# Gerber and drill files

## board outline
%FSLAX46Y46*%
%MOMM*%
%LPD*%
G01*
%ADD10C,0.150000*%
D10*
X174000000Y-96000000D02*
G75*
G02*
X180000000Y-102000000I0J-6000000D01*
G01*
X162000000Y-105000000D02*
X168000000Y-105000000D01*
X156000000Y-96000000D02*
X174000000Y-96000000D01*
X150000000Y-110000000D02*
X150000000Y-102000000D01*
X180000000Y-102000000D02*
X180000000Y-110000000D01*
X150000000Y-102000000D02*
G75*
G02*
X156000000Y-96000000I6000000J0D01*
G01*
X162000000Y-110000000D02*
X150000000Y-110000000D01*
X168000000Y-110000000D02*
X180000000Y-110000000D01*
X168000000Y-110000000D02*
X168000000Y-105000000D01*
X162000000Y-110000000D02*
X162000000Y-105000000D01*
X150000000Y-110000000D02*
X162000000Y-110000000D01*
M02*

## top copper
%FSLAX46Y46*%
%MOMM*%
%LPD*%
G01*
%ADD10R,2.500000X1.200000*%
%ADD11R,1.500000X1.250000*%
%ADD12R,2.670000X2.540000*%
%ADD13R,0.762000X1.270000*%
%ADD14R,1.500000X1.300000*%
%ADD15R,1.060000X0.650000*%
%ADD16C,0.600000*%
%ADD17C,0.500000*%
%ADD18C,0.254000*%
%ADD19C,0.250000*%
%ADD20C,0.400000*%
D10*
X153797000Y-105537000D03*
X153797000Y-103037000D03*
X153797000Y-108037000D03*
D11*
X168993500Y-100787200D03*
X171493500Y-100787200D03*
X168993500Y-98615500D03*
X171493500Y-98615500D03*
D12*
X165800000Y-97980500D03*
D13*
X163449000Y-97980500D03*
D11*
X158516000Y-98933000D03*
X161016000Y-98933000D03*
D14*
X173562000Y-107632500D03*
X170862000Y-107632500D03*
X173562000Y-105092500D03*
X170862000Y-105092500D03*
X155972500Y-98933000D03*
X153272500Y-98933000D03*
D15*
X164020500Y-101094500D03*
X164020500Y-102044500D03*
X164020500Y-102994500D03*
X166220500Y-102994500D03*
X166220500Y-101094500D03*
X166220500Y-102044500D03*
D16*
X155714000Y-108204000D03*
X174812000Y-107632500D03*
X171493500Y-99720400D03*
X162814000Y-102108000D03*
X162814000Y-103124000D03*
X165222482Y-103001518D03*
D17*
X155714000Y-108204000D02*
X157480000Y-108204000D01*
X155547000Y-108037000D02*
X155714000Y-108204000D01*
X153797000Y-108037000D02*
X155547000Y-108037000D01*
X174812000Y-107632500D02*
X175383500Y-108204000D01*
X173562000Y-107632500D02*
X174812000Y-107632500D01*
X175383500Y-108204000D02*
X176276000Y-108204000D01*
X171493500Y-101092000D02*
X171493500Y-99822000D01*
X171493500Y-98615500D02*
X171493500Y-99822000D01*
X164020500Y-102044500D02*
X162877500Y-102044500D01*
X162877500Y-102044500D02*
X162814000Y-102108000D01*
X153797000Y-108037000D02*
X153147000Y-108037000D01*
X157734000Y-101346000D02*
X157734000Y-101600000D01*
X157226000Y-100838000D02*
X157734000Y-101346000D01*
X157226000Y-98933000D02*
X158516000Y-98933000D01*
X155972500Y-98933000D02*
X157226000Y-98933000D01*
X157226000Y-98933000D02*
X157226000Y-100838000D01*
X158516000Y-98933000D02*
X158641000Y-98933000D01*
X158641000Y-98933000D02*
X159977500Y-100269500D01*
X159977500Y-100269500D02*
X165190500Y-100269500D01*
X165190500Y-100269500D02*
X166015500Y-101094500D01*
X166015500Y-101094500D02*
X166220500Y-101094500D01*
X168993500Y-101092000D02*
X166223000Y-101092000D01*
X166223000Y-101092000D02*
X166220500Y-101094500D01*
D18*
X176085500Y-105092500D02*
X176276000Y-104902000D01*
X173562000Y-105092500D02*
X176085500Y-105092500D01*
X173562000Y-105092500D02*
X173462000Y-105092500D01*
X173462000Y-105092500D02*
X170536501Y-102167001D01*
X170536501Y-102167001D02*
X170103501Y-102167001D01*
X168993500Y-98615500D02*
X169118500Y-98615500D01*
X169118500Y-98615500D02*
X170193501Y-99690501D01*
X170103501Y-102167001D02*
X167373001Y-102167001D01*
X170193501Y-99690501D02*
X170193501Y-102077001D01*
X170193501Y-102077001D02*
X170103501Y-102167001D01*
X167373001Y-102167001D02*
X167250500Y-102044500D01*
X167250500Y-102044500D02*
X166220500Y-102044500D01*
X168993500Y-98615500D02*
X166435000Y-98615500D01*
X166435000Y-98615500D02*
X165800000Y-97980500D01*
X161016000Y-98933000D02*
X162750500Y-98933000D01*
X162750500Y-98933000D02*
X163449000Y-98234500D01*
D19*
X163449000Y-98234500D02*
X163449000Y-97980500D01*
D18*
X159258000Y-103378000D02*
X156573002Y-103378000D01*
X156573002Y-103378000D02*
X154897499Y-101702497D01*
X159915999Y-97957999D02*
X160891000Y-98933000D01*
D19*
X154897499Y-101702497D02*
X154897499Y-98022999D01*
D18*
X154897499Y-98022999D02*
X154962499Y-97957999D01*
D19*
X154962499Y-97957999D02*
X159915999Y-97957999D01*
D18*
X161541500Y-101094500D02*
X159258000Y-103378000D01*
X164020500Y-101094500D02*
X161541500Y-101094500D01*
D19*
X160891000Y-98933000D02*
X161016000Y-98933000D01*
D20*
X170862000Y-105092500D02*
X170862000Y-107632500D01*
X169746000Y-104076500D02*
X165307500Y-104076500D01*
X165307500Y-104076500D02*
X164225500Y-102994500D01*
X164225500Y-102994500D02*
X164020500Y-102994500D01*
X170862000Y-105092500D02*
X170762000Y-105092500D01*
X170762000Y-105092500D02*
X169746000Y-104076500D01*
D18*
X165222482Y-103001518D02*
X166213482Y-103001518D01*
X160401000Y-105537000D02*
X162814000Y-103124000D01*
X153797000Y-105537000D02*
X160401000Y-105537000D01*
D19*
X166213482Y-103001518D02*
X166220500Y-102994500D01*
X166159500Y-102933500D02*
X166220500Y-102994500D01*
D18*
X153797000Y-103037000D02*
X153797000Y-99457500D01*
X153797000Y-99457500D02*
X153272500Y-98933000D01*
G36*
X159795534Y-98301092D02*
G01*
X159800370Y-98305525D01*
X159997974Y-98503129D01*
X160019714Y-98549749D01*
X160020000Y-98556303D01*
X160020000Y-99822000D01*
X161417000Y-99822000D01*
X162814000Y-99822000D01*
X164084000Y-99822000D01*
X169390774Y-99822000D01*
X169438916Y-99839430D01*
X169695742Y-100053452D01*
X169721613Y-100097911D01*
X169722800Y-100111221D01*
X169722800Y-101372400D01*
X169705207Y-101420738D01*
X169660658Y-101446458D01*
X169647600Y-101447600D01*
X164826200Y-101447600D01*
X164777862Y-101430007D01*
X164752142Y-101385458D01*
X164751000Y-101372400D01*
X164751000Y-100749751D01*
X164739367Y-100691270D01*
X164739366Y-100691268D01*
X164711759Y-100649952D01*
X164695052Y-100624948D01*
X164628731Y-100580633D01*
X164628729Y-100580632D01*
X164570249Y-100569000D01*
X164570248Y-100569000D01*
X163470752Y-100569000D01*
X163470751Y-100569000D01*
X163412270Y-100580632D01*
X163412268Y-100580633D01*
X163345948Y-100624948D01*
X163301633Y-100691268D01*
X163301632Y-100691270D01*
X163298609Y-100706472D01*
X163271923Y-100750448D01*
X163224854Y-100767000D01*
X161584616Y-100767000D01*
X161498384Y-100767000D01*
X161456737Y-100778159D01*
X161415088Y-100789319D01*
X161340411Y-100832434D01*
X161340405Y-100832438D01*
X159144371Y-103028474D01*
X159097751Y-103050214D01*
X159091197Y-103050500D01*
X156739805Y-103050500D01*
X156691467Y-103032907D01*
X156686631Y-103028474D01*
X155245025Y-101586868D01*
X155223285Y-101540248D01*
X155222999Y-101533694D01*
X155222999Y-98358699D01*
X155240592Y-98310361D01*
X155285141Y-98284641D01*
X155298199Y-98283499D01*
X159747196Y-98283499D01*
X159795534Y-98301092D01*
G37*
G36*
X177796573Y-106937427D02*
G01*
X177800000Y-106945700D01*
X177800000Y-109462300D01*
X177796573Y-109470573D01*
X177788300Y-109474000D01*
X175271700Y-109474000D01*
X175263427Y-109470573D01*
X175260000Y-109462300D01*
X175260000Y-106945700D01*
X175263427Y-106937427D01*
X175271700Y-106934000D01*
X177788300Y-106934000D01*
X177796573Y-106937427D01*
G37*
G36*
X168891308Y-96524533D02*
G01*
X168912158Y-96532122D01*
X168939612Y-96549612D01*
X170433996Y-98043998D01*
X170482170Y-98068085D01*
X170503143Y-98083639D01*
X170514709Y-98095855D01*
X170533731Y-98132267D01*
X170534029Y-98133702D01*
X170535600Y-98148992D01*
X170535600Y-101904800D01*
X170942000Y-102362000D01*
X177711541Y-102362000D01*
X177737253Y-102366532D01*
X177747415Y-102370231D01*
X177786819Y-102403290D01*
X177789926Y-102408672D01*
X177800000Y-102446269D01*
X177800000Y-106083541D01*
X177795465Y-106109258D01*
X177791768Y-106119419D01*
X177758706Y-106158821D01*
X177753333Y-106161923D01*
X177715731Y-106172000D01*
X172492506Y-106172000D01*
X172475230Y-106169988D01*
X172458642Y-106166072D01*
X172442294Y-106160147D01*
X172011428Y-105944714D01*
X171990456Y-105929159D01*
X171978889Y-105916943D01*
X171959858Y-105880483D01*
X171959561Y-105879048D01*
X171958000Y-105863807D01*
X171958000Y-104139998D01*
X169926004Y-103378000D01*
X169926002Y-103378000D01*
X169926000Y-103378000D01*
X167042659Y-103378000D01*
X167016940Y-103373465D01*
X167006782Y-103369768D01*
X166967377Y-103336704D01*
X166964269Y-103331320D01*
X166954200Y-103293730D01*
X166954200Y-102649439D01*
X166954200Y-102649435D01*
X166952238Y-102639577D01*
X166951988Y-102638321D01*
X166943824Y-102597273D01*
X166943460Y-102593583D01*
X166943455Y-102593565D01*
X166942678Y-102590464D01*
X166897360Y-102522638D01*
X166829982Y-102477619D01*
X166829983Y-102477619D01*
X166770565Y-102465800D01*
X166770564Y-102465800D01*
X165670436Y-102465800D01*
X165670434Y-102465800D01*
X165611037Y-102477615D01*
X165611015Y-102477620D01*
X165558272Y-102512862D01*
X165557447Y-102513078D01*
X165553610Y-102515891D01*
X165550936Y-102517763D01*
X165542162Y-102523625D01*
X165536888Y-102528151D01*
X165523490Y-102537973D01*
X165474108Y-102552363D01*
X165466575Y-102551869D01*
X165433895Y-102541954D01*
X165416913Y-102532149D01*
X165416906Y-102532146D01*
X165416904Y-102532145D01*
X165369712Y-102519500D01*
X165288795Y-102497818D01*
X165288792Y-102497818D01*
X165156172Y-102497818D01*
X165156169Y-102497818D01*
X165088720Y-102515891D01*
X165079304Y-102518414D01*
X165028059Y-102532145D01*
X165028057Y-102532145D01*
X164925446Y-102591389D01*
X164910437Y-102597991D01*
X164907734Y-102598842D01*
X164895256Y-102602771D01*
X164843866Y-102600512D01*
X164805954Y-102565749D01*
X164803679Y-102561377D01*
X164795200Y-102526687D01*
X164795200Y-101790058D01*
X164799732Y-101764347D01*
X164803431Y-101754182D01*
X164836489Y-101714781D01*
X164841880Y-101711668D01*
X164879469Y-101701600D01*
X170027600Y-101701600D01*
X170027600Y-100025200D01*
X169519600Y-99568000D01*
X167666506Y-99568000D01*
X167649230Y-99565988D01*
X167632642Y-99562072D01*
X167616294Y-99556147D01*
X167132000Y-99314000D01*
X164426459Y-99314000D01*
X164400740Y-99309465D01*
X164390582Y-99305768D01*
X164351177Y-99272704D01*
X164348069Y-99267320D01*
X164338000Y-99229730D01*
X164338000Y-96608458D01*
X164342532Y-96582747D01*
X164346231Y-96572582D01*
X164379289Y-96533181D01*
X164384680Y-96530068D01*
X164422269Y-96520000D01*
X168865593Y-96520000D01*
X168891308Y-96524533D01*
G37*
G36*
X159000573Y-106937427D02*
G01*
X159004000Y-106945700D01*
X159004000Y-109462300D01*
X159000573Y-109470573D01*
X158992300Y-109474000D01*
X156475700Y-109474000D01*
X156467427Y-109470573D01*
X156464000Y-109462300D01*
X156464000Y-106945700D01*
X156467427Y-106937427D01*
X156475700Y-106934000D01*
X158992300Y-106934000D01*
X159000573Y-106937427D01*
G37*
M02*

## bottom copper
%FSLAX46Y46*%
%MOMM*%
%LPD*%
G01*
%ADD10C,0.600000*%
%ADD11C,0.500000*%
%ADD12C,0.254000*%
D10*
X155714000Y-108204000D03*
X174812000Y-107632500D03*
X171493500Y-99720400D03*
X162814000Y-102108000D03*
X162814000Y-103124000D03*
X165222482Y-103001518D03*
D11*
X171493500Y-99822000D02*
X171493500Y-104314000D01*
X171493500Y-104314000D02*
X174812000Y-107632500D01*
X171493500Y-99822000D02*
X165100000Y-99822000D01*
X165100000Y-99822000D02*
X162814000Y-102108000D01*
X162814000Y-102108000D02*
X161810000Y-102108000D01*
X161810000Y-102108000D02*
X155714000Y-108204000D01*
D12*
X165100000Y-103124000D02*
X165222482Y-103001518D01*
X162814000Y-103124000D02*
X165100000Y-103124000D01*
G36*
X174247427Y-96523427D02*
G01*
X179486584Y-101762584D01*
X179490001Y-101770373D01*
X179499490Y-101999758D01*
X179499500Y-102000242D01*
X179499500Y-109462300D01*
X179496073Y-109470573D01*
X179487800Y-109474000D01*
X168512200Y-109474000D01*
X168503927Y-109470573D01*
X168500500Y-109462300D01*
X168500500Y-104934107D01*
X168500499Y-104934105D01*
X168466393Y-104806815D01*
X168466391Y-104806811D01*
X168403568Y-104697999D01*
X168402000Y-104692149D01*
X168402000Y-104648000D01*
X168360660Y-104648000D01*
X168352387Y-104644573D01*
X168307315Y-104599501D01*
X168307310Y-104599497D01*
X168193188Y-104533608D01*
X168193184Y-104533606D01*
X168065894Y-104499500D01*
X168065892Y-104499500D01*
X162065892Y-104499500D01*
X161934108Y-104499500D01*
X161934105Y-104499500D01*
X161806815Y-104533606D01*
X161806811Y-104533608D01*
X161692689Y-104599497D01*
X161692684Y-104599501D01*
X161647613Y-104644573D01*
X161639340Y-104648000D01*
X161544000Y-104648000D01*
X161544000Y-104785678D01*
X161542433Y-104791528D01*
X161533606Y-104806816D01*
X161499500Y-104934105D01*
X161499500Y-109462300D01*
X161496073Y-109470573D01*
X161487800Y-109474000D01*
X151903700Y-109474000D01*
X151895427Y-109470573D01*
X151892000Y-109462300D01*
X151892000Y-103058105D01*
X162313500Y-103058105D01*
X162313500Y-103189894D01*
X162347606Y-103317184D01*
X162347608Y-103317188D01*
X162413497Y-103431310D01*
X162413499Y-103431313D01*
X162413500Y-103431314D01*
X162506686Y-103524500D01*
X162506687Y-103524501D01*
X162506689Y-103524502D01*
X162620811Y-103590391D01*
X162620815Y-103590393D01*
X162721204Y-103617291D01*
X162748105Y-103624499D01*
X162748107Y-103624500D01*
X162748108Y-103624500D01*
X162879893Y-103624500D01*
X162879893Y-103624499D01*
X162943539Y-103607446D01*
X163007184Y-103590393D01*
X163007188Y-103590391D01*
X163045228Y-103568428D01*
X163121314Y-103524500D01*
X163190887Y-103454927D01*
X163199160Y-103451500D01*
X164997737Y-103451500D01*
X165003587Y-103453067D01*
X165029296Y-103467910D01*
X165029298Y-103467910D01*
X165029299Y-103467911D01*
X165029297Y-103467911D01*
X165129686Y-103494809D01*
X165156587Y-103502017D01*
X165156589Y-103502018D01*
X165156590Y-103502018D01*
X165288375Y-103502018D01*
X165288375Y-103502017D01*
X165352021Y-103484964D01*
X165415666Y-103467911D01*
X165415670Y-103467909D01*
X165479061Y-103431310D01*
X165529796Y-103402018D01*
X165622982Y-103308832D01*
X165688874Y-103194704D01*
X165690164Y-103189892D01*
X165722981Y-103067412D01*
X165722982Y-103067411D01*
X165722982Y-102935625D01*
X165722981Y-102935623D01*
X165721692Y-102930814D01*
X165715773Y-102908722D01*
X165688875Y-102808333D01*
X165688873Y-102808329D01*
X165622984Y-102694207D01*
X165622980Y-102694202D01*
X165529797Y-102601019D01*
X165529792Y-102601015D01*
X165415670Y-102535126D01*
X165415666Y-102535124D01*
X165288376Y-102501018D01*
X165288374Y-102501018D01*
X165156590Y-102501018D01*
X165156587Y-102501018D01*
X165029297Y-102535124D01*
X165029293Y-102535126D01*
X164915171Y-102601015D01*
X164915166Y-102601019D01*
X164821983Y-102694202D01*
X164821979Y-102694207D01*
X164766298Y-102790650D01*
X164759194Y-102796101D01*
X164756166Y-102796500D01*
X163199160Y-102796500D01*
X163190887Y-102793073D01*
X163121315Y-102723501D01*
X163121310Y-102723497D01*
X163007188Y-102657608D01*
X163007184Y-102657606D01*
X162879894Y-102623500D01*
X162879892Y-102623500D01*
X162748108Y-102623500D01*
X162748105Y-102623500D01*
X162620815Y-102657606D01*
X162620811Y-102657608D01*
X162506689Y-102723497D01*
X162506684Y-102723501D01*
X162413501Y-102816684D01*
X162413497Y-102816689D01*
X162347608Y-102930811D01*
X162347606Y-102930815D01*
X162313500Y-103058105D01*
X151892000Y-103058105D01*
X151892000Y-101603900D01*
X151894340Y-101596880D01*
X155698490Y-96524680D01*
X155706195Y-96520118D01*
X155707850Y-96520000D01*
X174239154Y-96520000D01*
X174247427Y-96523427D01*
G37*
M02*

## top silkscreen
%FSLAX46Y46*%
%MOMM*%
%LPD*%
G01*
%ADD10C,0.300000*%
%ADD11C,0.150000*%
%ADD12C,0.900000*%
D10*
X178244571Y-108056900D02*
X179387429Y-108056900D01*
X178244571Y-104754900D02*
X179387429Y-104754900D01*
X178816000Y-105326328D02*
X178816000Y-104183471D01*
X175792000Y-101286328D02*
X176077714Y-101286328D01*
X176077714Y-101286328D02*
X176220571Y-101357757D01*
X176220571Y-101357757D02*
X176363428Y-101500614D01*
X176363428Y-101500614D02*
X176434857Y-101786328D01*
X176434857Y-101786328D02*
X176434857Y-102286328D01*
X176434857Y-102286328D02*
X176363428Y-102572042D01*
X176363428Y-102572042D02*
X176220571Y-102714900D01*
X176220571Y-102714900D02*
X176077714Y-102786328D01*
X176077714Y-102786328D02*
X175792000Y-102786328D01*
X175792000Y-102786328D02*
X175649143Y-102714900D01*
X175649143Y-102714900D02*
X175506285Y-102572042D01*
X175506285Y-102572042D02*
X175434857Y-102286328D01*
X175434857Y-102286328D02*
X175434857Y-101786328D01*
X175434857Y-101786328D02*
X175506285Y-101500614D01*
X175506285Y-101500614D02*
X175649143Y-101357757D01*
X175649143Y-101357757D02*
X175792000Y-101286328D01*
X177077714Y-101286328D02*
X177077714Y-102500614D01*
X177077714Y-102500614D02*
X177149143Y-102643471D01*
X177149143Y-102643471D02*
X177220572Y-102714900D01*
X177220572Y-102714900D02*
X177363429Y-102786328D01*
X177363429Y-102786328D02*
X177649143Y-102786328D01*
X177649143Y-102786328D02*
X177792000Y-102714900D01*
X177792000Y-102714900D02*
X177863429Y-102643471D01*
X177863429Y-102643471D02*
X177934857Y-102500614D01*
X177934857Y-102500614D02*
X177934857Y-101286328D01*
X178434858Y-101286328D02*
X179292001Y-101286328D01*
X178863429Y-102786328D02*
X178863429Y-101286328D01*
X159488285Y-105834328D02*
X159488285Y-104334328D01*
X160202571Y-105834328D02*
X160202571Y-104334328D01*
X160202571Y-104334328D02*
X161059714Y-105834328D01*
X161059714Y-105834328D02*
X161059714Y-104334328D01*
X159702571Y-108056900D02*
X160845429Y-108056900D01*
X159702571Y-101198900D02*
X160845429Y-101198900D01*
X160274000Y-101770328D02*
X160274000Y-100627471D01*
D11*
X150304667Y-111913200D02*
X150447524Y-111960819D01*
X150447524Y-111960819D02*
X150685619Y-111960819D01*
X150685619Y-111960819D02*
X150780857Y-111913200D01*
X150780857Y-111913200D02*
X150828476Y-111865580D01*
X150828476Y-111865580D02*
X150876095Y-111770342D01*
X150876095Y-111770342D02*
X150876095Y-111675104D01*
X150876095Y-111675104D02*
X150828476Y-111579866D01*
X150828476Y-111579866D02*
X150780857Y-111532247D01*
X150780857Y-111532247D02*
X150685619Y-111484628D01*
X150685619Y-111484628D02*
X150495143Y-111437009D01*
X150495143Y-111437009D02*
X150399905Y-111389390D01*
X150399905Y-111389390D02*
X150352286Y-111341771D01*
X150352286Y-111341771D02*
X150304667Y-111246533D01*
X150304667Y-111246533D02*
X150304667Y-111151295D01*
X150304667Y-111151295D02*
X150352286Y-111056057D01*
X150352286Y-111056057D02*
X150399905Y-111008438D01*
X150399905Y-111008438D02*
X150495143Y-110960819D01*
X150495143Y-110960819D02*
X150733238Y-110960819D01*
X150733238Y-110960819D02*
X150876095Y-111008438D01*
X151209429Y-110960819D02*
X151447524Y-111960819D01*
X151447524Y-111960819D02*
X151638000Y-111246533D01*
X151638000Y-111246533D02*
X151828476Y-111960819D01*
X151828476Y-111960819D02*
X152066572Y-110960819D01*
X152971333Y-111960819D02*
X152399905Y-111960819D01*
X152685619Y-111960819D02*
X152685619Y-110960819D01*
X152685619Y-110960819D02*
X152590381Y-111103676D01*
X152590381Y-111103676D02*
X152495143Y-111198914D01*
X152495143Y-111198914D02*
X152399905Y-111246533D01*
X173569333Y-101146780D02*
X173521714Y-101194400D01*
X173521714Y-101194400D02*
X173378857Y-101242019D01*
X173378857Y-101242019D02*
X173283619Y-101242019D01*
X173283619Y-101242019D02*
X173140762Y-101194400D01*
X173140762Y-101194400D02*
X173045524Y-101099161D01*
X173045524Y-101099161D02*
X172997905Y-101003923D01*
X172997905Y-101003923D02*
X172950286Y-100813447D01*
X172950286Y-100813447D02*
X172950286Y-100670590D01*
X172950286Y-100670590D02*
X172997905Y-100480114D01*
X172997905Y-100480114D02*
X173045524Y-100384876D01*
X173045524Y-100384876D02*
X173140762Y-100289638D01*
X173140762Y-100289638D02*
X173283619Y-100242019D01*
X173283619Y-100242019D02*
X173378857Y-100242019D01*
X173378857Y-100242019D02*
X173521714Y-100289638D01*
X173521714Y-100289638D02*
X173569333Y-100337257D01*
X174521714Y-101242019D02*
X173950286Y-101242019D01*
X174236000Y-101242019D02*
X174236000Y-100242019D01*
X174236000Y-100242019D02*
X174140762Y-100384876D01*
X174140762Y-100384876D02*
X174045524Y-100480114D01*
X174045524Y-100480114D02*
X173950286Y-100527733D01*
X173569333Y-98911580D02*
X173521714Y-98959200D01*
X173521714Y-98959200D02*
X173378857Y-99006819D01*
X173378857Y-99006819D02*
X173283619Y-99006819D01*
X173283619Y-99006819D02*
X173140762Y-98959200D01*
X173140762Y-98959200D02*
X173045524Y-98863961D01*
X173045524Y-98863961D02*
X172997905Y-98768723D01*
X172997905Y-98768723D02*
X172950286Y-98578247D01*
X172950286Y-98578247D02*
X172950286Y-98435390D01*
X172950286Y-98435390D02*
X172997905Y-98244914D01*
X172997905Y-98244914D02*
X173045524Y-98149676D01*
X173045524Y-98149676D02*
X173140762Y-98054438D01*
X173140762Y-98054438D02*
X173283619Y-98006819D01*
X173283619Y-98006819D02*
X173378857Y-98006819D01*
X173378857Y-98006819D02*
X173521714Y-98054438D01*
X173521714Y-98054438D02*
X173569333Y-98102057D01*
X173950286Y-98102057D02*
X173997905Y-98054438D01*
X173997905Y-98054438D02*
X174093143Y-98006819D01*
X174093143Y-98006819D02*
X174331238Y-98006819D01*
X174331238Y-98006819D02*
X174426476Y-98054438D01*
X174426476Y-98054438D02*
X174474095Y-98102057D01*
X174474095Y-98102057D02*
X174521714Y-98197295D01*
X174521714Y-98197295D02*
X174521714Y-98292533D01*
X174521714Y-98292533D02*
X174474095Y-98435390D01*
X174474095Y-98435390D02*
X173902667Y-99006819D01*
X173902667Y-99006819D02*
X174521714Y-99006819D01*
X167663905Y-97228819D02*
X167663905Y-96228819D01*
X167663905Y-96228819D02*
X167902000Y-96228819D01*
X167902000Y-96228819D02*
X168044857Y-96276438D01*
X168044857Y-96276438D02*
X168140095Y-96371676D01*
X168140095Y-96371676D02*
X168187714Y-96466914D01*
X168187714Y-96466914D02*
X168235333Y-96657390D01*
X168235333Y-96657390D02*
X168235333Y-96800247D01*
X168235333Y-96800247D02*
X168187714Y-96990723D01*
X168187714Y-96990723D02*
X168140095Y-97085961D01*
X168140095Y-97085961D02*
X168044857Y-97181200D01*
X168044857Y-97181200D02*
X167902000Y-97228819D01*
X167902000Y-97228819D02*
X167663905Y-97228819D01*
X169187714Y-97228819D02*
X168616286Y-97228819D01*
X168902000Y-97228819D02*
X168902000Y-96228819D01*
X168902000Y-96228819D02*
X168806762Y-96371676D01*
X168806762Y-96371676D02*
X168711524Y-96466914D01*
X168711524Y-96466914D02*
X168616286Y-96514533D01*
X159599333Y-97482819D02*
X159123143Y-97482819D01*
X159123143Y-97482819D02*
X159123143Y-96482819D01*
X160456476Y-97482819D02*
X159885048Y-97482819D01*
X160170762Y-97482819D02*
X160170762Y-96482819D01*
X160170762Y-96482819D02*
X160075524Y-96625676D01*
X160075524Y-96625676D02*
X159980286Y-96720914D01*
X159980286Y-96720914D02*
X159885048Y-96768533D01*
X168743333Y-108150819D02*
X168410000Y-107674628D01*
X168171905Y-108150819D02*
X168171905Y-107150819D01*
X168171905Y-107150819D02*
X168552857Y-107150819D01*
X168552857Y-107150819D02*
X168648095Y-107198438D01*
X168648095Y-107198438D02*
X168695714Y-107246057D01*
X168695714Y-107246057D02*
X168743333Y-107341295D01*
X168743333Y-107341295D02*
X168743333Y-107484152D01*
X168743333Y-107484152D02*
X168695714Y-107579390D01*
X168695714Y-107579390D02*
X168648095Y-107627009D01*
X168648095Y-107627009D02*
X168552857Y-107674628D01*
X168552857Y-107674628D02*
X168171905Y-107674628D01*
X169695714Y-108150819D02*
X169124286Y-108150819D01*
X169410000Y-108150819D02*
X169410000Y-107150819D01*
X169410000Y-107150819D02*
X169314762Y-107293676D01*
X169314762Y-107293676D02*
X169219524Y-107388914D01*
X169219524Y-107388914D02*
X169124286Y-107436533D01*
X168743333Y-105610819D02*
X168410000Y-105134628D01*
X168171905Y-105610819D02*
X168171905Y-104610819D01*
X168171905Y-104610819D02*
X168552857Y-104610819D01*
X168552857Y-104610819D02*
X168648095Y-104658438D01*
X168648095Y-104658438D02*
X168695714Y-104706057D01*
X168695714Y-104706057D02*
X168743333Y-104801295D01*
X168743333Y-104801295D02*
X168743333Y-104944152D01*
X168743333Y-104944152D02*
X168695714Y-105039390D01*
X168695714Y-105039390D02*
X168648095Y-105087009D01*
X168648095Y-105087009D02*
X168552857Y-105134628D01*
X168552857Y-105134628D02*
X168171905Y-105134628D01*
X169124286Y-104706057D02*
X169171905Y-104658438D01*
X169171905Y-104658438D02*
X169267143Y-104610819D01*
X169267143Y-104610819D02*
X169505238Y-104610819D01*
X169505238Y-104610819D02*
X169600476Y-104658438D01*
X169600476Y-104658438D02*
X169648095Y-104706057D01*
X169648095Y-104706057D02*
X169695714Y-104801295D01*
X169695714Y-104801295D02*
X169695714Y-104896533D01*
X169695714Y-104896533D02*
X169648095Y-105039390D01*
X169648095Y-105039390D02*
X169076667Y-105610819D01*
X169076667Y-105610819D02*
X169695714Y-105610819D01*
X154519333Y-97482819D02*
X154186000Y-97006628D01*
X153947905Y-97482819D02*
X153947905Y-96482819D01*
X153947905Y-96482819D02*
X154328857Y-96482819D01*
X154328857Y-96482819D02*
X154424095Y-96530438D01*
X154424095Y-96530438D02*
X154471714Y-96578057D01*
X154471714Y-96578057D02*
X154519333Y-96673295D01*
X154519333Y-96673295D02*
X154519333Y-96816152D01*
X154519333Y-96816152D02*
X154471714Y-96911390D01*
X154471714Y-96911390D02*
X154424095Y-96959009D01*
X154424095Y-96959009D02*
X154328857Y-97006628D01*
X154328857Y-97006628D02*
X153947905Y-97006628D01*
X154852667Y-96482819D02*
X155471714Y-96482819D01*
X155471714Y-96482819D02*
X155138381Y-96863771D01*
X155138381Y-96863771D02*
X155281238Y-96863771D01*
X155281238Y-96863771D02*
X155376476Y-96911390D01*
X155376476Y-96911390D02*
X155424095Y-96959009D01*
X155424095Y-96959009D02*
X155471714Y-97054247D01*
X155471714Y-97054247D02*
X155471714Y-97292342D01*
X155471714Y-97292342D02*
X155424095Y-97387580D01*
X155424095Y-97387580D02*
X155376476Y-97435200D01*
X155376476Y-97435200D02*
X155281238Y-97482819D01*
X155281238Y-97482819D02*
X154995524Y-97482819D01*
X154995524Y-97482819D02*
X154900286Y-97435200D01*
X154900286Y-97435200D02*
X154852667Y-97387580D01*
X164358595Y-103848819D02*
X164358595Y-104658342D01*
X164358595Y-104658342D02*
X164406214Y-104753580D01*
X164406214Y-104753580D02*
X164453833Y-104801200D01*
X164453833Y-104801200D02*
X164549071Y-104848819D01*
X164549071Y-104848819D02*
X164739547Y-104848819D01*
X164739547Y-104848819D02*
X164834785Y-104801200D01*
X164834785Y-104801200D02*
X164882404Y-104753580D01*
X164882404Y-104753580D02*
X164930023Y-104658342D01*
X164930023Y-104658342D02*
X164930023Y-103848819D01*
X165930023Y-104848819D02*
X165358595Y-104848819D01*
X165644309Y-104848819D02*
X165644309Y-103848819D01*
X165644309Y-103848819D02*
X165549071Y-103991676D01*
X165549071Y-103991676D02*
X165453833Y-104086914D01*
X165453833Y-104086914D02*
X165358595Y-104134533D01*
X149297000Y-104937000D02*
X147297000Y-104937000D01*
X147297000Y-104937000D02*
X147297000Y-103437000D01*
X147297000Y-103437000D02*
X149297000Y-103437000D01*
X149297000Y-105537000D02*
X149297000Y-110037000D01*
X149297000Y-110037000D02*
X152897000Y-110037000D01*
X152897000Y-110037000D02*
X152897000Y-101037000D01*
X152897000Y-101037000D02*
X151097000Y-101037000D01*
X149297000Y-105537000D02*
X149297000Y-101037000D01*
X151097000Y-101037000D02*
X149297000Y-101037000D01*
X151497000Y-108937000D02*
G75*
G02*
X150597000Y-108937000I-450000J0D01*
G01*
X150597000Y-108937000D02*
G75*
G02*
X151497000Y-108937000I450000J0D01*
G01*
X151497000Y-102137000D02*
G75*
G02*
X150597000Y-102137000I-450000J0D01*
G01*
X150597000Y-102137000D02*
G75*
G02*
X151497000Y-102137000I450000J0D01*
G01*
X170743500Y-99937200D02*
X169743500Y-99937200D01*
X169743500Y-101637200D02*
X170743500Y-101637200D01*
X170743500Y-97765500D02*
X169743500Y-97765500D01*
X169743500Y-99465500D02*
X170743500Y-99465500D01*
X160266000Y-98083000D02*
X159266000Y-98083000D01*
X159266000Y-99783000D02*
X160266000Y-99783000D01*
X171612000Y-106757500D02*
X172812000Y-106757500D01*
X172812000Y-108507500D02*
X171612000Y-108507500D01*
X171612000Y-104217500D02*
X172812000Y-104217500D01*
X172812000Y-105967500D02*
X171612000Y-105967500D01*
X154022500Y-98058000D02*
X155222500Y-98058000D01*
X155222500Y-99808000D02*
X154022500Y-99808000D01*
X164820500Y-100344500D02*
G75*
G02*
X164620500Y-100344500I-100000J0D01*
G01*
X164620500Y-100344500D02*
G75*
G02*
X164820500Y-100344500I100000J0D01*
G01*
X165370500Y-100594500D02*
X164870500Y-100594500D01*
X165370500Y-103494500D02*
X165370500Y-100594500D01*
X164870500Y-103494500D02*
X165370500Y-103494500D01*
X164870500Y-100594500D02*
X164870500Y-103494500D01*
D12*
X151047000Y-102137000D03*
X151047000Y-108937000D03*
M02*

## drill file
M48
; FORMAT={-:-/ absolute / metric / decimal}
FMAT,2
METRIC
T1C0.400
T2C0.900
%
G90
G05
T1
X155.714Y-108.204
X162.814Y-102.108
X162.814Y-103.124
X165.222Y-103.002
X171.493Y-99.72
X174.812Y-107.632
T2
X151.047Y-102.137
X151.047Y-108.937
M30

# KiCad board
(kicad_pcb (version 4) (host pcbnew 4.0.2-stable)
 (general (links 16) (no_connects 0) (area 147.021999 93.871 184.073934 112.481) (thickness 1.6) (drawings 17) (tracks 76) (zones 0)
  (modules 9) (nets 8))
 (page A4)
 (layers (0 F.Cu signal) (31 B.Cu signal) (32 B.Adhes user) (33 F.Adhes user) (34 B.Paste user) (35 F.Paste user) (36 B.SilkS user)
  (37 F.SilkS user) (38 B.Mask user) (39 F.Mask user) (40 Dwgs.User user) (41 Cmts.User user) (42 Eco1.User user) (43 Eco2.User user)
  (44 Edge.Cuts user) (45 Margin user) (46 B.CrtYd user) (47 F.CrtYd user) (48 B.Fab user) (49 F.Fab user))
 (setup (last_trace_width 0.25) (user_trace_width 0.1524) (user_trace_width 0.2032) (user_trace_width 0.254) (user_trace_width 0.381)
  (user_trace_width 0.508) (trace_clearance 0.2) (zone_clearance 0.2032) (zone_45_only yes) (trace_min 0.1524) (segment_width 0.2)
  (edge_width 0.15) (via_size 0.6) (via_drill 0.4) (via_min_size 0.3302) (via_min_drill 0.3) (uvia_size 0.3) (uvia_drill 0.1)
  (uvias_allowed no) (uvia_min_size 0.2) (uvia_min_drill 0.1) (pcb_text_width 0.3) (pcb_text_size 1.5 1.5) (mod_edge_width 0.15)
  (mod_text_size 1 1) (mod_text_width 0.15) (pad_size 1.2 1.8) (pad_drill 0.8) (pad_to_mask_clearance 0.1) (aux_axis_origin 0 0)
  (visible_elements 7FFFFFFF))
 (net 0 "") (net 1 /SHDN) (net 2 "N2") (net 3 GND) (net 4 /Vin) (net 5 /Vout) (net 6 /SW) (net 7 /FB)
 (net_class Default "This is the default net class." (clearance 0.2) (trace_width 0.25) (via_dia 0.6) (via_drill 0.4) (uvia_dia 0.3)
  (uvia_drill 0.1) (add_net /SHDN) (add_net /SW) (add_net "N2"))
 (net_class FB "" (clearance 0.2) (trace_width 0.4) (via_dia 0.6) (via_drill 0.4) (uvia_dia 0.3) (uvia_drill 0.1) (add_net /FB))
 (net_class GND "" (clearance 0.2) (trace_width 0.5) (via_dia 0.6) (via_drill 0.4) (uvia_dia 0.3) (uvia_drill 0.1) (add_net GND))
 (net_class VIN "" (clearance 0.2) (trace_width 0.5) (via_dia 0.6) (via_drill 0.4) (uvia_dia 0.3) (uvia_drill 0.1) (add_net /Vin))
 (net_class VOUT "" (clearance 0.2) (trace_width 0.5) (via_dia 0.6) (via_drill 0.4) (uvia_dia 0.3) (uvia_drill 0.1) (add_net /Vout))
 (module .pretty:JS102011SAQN (layer F.Cu) (at 153.797 105.537 270)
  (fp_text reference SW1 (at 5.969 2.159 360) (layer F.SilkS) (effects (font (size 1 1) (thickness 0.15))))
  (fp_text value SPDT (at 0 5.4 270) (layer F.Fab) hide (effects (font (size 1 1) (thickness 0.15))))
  (fp_line (start -0.6 4.5) (end -0.6 6.5) (layer F.SilkS) (width 0.15))
  (fp_line (start -0.6 6.5) (end -2.1 6.5) (layer F.SilkS) (width 0.15))
  (fp_line (start -2.1 6.5) (end -2.1 4.5) (layer F.SilkS) (width 0.15))
  (fp_line (start 0 4.5) (end 4.5 4.5) (layer F.SilkS) (width 0.15))
  (fp_line (start 4.5 4.5) (end 4.5 0.9) (layer F.SilkS) (width 0.15))
  (fp_line (start 4.5 0.9) (end -4.5 0.9) (layer F.SilkS) (width 0.15))
  (fp_line (start -4.5 0.9) (end -4.5 2.7) (layer F.SilkS) (width 0.15))
  (fp_line (start 0 4.5) (end -4.5 4.5) (layer F.SilkS) (width 0.15))
  (fp_line (start -4.5 2.7) (end -4.5 4.5) (layer F.SilkS) (width 0.15))
  (fp_circle (center 3.4 2.75) (end 3.85 2.75) (layer F.SilkS) (width 0.15))
  (fp_circle (center -3.4 2.75) (end -3.85 2.75) (layer F.SilkS) (width 0.15))
  (pad 2 smd rect (at 0 0 270) (size 1.2 2.5) (layers F.Cu F.Paste F.Mask) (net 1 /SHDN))
  (pad 1 smd rect (at -2.5 0 270) (size 1.2 2.5) (layers F.Cu F.Paste F.Mask) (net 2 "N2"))
  (pad 3 smd rect (at 2.5 0 270) (size 1.2 2.5) (layers F.Cu F.Paste F.Mask) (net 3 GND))
  (pad "" np_thru_hole circle (at -3.4 2.75 270) (size 0.9 0.9) (drill 0.9) (layers *.Cu *.Mask F.SilkS))
  (pad "" np_thru_hole circle (at 3.4 2.75 270) (size 0.9 0.9) (drill 0.9) (layers *.Cu *.Mask F.SilkS)))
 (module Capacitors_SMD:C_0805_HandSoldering (layer F.Cu) (at 170.2435 100.7872)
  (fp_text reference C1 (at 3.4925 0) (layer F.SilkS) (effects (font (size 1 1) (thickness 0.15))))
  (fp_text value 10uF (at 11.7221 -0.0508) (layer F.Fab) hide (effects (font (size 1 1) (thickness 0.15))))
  (fp_line (start 0.5 -0.85) (end -0.5 -0.85) (layer F.SilkS) (width 0.15))
  (fp_line (start -0.5 0.85) (end 0.5 0.85) (layer F.SilkS) (width 0.15))
  (pad 1 smd rect (at -1.25 0) (size 1.5 1.25) (layers F.Cu F.Paste F.Mask) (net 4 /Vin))
  (pad 2 smd rect (at 1.25 0) (size 1.5 1.25) (layers F.Cu F.Paste F.Mask) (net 3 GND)))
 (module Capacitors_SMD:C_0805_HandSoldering (layer F.Cu) (at 170.2435 98.6155)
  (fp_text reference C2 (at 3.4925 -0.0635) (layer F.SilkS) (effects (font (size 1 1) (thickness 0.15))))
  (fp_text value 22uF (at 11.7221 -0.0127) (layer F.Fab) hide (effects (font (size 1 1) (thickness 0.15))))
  (fp_line (start 0.5 -0.85) (end -0.5 -0.85) (layer F.SilkS) (width 0.15))
  (fp_line (start -0.5 0.85) (end 0.5 0.85) (layer F.SilkS) (width 0.15))
  (pad 1 smd rect (at -1.25 0) (size 1.5 1.25) (layers F.Cu F.Paste F.Mask) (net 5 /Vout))
  (pad 2 smd rect (at 1.25 0) (size 1.5 1.25) (layers F.Cu F.Paste F.Mask) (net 3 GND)))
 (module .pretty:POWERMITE (layer F.Cu) (at 164.1475 97.9805 180)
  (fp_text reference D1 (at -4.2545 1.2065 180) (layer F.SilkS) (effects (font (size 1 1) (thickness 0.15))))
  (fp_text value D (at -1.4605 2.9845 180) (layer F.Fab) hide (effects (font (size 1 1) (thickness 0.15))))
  (pad 1 smd rect (at -1.6525 0 180) (size 2.67 2.54) (layers F.Cu F.Paste F.Mask) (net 5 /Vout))
  (pad 2 smd rect (at 0.6985 0 180) (size 0.762 1.27) (layers F.Cu F.Paste F.Mask) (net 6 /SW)))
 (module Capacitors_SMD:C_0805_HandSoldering (layer F.Cu) (at 159.766 98.933)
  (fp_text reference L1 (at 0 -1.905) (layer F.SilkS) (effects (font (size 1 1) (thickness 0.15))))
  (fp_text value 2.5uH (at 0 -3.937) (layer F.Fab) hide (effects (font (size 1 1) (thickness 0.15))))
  (fp_line (start 0.5 -0.85) (end -0.5 -0.85) (layer F.SilkS) (width 0.15))
  (fp_line (start -0.5 0.85) (end 0.5 0.85) (layer F.SilkS) (width 0.15))
  (pad 1 smd rect (at -1.25 0) (size 1.5 1.25) (layers F.Cu F.Paste F.Mask) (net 4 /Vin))
  (pad 2 smd rect (at 1.25 0) (size 1.5 1.25) (layers F.Cu F.Paste F.Mask) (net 6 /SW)))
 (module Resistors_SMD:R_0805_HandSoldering (layer F.Cu) (at 172.212 107.6325 180)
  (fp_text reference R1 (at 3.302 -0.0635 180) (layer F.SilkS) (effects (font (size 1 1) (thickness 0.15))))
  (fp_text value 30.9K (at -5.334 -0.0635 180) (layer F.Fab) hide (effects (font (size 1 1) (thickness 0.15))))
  (fp_line (start 0.6 0.875) (end -0.6 0.875) (layer F.SilkS) (width 0.15))
  (fp_line (start -0.6 -0.875) (end 0.6 -0.875) (layer F.SilkS) (width 0.15))
  (pad 1 smd rect (at -1.35 0 180) (size 1.5 1.3) (layers F.Cu F.Paste F.Mask) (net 3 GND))
  (pad 2 smd rect (at 1.35 0 180) (size 1.5 1.3) (layers F.Cu F.Paste F.Mask) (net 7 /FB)))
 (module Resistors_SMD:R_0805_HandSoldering (layer F.Cu) (at 172.212 105.0925 180)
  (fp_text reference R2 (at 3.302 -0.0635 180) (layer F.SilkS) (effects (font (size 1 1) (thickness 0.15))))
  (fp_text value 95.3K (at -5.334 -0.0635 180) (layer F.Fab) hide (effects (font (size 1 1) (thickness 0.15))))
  (fp_line (start 0.6 0.875) (end -0.6 0.875) (layer F.SilkS) (width 0.15))
  (fp_line (start -0.6 -0.875) (end 0.6 -0.875) (layer F.SilkS) (width 0.15))
  (pad 1 smd rect (at -1.35 0 180) (size 1.5 1.3) (layers F.Cu F.Paste F.Mask) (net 5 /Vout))
  (pad 2 smd rect (at 1.35 0 180) (size 1.5 1.3) (layers F.Cu F.Paste F.Mask) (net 7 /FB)))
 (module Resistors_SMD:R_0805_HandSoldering (layer F.Cu) (at 154.6225 98.933 180)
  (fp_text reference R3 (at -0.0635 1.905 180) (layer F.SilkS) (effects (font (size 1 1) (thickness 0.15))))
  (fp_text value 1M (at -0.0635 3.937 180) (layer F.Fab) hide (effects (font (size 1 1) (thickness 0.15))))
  (fp_line (start 0.6 0.875) (end -0.6 0.875) (layer F.SilkS) (width 0.15))
  (fp_line (start -0.6 -0.875) (end 0.6 -0.875) (layer F.SilkS) (width 0.15))
  (pad 1 smd rect (at -1.35 0 180) (size 1.5 1.3) (layers F.Cu F.Paste F.Mask) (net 4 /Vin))
  (pad 2 smd rect (at 1.35 0 180) (size 1.5 1.3) (layers F.Cu F.Paste F.Mask) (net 2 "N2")))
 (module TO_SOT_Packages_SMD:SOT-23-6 (layer F.Cu) (at 165.1205 102.0445)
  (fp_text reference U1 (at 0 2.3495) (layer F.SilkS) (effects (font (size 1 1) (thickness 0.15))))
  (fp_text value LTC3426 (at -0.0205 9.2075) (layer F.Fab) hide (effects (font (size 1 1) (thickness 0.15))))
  (fp_circle (center -0.4 -1.7) (end -0.3 -1.7) (layer F.SilkS) (width 0.15))
  (fp_line (start 0.25 -1.45) (end -0.25 -1.45) (layer F.SilkS) (width 0.15))
  (fp_line (start 0.25 1.45) (end 0.25 -1.45) (layer F.SilkS) (width 0.15))
  (fp_line (start -0.25 1.45) (end 0.25 1.45) (layer F.SilkS) (width 0.15))
  (fp_line (start -0.25 -1.45) (end -0.25 1.45) (layer F.SilkS) (width 0.15))
  (pad 1 smd rect (at -1.1 -0.95) (size 1.06 0.65) (layers F.Cu F.Paste F.Mask) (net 6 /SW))
  (pad 2 smd rect (at -1.1 0) (size 1.06 0.65) (layers F.Cu F.Paste F.Mask) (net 3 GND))
  (pad 3 smd rect (at -1.1 0.95) (size 1.06 0.65) (layers F.Cu F.Paste F.Mask) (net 7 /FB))
  (pad 4 smd rect (at 1.1 0.95) (size 1.06 0.65) (layers F.Cu F.Paste F.Mask) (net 1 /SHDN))
  (pad 6 smd rect (at 1.1 -0.95) (size 1.06 0.65) (layers F.Cu F.Paste F.Mask) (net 4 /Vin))
  (pad 5 smd rect (at 1.1 0) (size 1.06 0.65) (layers F.Cu F.Paste F.Mask) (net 5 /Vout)))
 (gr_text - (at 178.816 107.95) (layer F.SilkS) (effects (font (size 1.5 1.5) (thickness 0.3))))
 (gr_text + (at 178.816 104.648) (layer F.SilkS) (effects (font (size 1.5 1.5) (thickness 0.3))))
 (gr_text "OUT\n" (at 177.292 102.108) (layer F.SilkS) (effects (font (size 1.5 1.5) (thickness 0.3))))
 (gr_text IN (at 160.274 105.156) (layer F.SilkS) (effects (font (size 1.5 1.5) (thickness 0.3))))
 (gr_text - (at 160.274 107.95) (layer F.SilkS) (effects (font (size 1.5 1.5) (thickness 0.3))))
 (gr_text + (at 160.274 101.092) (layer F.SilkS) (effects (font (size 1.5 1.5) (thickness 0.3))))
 (gr_arc (start 174 102) (end 174 96) (angle 90) (layer Edge.Cuts) (width 0.15))
 (gr_line (start 162 105) (end 168 105) (angle 90) (layer Edge.Cuts) (width 0.15))
 (gr_line (start 156 96) (end 174 96) (angle 90) (layer Edge.Cuts) (width 0.15))
 (gr_line (start 150 110) (end 150 102) (angle 90) (layer Edge.Cuts) (width 0.15))
 (gr_line (start 180 102) (end 180 110) (angle 90) (layer Edge.Cuts) (width 0.15))
 (gr_arc (start 156 102) (end 150 102) (angle 90) (layer Edge.Cuts) (width 0.15))
 (gr_line (start 162 110) (end 150 110) (angle 90) (layer Edge.Cuts) (width 0.15))
 (gr_line (start 168 110) (end 180 110) (angle 90) (layer Edge.Cuts) (width 0.15))
 (gr_line (start 168 110) (end 168 105) (angle 90) (layer Edge.Cuts) (width 0.15))
 (gr_line (start 162 110) (end 162 105) (angle 90) (layer Edge.Cuts) (width 0.15))
 (gr_line (start 150 110) (end 162 110) (angle 90) (layer Edge.Cuts) (width 0.15))
 (segment (start 155.714 108.204) (end 157.48 108.204) (width 0.5) (layer F.Cu) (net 3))
 (via (at 155.714 108.204) (size 0.6) (drill 0.4) (layers F.Cu B.Cu) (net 3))
 (segment (start 155.547 108.037) (end 155.714 108.204) (width 0.5) (layer F.Cu) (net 3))
 (segment (start 153.797 108.037) (end 155.547 108.037) (width 0.5) (layer F.Cu) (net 3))
 (via (at 174.812 107.6325) (size 0.6) (drill 0.4) (layers F.Cu B.Cu) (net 3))
 (segment (start 174.812 107.6325) (end 175.3835 108.204) (width 0.5) (layer F.Cu) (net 3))
 (segment (start 173.562 107.6325) (end 174.812 107.6325) (width 0.5) (layer F.Cu) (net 3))
 (segment (start 175.3835 108.204) (end 176.276 108.204) (width 0.5) (layer F.Cu) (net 3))
 (segment (start 171.4935 99.822) (end 171.4935 104.314) (width 0.5) (layer B.Cu) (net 3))
 (segment (start 171.4935 104.314) (end 174.812 107.6325) (width 0.5) (layer B.Cu) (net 3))
 (segment (start 171.4935 99.822) (end 165.1 99.822) (width 0.5) (layer B.Cu) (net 3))
 (segment (start 165.1 99.822) (end 162.814 102.108) (width 0.5) (layer B.Cu) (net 3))
 (segment (start 162.814 102.108) (end 161.81 102.108) (width 0.5) (layer B.Cu) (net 3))
 (segment (start 161.81 102.108) (end 155.714 108.204) (width 0.5) (layer B.Cu) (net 3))
 (segment (start 171.4935 101.092) (end 171.4935 99.822) (width 0.5) (layer F.Cu) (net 3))
 (segment (start 171.4935 98.6155) (end 171.4935 99.822) (width 0.5) (layer F.Cu) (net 3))
 (via (at 171.4935 99.7204) (size 0.6) (drill 0.4) (layers F.Cu B.Cu) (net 3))
 (segment (start 164.0205 102.0445) (end 162.8775 102.0445) (width 0.5) (layer F.Cu) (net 3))
 (segment (start 162.8775 102.0445) (end 162.814 102.108) (width 0.5) (layer F.Cu) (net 3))
 (via (at 162.814 102.108) (size 0.6) (drill 0.4) (layers F.Cu B.Cu) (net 3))
 (segment (start 153.797 108.037) (end 153.147 108.037) (width 0.5) (layer F.Cu) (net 3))
 (segment (start 157.734 101.346) (end 157.734 101.6) (width 0.5) (layer F.Cu) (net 4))
 (segment (start 157.226 100.838) (end 157.734 101.346) (width 0.5) (layer F.Cu) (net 4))
 (segment (start 157.226 98.933) (end 158.516 98.933) (width 0.5) (layer F.Cu) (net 4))
 (segment (start 155.9725 98.933) (end 157.226 98.933) (width 0.5) (layer F.Cu) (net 4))
 (segment (start 157.226 98.933) (end 157.226 100.838) (width 0.5) (layer F.Cu) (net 4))
 (segment (start 158.516 98.933) (end 158.641 98.933) (width 0.5) (layer F.Cu) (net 4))
 (segment (start 158.641 98.933) (end 159.9775 100.2695) (width 0.5) (layer F.Cu) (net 4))
 (segment (start 159.9775 100.2695) (end 165.1905 100.2695) (width 0.5) (layer F.Cu) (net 4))
 (segment (start 165.1905 100.2695) (end 166.0155 101.0945) (width 0.5) (layer F.Cu) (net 4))
 (segment (start 166.0155 101.0945) (end 166.2205 101.0945) (width 0.5) (layer F.Cu) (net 4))
 (segment (start 168.9935 101.092) (end 166.223 101.092) (width 0.5) (layer F.Cu) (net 4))
 (segment (start 166.223 101.092) (end 166.2205 101.0945) (width 0.5) (layer F.Cu) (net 4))
 (segment (start 176.0855 105.0925) (end 176.276 104.902) (width 0.254) (layer F.Cu) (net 5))
 (segment (start 173.562 105.0925) (end 176.0855 105.0925) (width 0.254) (layer F.Cu) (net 5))
 (segment (start 173.562 105.0925) (end 173.462 105.0925) (width 0.254) (layer F.Cu) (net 5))
 (segment (start 173.462 105.0925) (end 170.536501 102.167001) (width 0.254) (layer F.Cu) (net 5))
 (segment (start 170.536501 102.167001) (end 170.103501 102.167001) (width 0.254) (layer F.Cu) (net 5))
 (segment (start 168.9935 98.6155) (end 169.1185 98.6155) (width 0.254) (layer F.Cu) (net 5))
 (segment (start 169.1185 98.6155) (end 170.193501 99.690501) (width 0.254) (layer F.Cu) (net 5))
 (segment (start 170.103501 102.167001) (end 167.373001 102.167001) (width 0.254) (layer F.Cu) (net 5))
 (segment (start 170.193501 99.690501) (end 170.193501 102.077001) (width 0.254) (layer F.Cu) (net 5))
 (segment (start 170.193501 102.077001) (end 170.103501 102.167001) (width 0.254) (layer F.Cu) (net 5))
 (segment (start 167.373001 102.167001) (end 167.2505 102.0445) (width 0.254) (layer F.Cu) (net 5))
 (segment (start 167.2505 102.0445) (end 166.2205 102.0445) (width 0.254) (layer F.Cu) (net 5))
 (segment (start 168.9935 98.6155) (end 166.435 98.6155) (width 0.254) (layer F.Cu) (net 5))
 (segment (start 166.435 98.6155) (end 165.8 97.9805) (width 0.254) (layer F.Cu) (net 5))
 (segment (start 161.016 98.933) (end 162.7505 98.933) (width 0.254) (layer F.Cu) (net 6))
 (segment (start 162.7505 98.933) (end 163.449 98.2345) (width 0.254) (layer F.Cu) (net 6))
 (segment (start 163.449 98.2345) (end 163.449 97.9805) (width 0.25) (layer F.Cu) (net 6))
 (segment (start 159.258 103.378) (end 156.573002 103.378) (width 0.254) (layer F.Cu) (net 6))
 (segment (start 156.573002 103.378) (end 154.897499 101.702497) (width 0.254) (layer F.Cu) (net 6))
 (segment (start 159.915999 97.957999) (end 160.891 98.933) (width 0.254) (layer F.Cu) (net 6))
 (segment (start 154.897499 101.702497) (end 154.897499 98.022999) (width 0.25) (layer F.Cu) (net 6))
 (segment (start 154.897499 98.022999) (end 154.962499 97.957999) (width 0.254) (layer F.Cu) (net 6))
 (segment (start 154.962499 97.957999) (end 159.915999 97.957999) (width 0.25) (layer F.Cu) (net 6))
 (segment (start 161.5415 101.0945) (end 159.258 103.378) (width 0.254) (layer F.Cu) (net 6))
 (segment (start 164.0205 101.0945) (end 161.5415 101.0945) (width 0.254) (layer F.Cu) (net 6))
 (segment (start 160.891 98.933) (end 161.016 98.933) (width 0.25) (layer F.Cu) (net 6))
 (segment (start 170.862 105.0925) (end 170.862 107.6325) (width 0.4) (layer F.Cu) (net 7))
 (segment (start 169.746 104.0765) (end 165.3075 104.0765) (width 0.4) (layer F.Cu) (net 7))
 (segment (start 165.3075 104.0765) (end 164.2255 102.9945) (width 0.4) (layer F.Cu) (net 7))
 (segment (start 164.2255 102.9945) (end 164.0205 102.9945) (width 0.4) (layer F.Cu) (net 7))
 (segment (start 170.862 105.0925) (end 170.762 105.0925) (width 0.4) (layer F.Cu) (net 7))
 (segment (start 170.762 105.0925) (end 169.746 104.0765) (width 0.4) (layer F.Cu) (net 7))
 (segment (start 165.222482 103.001518) (end 166.213482 103.001518) (width 0.254) (layer F.Cu) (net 1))
 (via (at 162.814 103.124) (size 0.6) (drill 0.4) (layers F.Cu B.Cu) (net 1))
 (segment (start 160.401 105.537) (end 162.814 103.124) (width 0.254) (layer F.Cu) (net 1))
 (segment (start 153.797 105.537) (end 160.401 105.537) (width 0.254) (layer F.Cu) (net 1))
 (via (at 165.222482 103.001518) (size 0.6) (drill 0.4) (layers F.Cu B.Cu) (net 1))
 (segment (start 165.1 103.124) (end 165.222482 103.001518) (width 0.254) (layer B.Cu) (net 1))
 (segment (start 162.814 103.124) (end 165.1 103.124) (width 0.254) (layer B.Cu) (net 1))
 (segment (start 166.213482 103.001518) (end 166.2205 102.9945) (width 0.25) (layer F.Cu) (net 1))
 (segment (start 166.1595 102.9335) (end 166.2205 102.9945) (width 0.25) (layer F.Cu) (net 1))
 (segment (start 153.797 103.037) (end 153.797 99.4575) (width 0.254) (layer F.Cu) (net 2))
 (segment (start 153.797 99.4575) (end 153.2725 98.933) (width 0.254) (layer F.Cu) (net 2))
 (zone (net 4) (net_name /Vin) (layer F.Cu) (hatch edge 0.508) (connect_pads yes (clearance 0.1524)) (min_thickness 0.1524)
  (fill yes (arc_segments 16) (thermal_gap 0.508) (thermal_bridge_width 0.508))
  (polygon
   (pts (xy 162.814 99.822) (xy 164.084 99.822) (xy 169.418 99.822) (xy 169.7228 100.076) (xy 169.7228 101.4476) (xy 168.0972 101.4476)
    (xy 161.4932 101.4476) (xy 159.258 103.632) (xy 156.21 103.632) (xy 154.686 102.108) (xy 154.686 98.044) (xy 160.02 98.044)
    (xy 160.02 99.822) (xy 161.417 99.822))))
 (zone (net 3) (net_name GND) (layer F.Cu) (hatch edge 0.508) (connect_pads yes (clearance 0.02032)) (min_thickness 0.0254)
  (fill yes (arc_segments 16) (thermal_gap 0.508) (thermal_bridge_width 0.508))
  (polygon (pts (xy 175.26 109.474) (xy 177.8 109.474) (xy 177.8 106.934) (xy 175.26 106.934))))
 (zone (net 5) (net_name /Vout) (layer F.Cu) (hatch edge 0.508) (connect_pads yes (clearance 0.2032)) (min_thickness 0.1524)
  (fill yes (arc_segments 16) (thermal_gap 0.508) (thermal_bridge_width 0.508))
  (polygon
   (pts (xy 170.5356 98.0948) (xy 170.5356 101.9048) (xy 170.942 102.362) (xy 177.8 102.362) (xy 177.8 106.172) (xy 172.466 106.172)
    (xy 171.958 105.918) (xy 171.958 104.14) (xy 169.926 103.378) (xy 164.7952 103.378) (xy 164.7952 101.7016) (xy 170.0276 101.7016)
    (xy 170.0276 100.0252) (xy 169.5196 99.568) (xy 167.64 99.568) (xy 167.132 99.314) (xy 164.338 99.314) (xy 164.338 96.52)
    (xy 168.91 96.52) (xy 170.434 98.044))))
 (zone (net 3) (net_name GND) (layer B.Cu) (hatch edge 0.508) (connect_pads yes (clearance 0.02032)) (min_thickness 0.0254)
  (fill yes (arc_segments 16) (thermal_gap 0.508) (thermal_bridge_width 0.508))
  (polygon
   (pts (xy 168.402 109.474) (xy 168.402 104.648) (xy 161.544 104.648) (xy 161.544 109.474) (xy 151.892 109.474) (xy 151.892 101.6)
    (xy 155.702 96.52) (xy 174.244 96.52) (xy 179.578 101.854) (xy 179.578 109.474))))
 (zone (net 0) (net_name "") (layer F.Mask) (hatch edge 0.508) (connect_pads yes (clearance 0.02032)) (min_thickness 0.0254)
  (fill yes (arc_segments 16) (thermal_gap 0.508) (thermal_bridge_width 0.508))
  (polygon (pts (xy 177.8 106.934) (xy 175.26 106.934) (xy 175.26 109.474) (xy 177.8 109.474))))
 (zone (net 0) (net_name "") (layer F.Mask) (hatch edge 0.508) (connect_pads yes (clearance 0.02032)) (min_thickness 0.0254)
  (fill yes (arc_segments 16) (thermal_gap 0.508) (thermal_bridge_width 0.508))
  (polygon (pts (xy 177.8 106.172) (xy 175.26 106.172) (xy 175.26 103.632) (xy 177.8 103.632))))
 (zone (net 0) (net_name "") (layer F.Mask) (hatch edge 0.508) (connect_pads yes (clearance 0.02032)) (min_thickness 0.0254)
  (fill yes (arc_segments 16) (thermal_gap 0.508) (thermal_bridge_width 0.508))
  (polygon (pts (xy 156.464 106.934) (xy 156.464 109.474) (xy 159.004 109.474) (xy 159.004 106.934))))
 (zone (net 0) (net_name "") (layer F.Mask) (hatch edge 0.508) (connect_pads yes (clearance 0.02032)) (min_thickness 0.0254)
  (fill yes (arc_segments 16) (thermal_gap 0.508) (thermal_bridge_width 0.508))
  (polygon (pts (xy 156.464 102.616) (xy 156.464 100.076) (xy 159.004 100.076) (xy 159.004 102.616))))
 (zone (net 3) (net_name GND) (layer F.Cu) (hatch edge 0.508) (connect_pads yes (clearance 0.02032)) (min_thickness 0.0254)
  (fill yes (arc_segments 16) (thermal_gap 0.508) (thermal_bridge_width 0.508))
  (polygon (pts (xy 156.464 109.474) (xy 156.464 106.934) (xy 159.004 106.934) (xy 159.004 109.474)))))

